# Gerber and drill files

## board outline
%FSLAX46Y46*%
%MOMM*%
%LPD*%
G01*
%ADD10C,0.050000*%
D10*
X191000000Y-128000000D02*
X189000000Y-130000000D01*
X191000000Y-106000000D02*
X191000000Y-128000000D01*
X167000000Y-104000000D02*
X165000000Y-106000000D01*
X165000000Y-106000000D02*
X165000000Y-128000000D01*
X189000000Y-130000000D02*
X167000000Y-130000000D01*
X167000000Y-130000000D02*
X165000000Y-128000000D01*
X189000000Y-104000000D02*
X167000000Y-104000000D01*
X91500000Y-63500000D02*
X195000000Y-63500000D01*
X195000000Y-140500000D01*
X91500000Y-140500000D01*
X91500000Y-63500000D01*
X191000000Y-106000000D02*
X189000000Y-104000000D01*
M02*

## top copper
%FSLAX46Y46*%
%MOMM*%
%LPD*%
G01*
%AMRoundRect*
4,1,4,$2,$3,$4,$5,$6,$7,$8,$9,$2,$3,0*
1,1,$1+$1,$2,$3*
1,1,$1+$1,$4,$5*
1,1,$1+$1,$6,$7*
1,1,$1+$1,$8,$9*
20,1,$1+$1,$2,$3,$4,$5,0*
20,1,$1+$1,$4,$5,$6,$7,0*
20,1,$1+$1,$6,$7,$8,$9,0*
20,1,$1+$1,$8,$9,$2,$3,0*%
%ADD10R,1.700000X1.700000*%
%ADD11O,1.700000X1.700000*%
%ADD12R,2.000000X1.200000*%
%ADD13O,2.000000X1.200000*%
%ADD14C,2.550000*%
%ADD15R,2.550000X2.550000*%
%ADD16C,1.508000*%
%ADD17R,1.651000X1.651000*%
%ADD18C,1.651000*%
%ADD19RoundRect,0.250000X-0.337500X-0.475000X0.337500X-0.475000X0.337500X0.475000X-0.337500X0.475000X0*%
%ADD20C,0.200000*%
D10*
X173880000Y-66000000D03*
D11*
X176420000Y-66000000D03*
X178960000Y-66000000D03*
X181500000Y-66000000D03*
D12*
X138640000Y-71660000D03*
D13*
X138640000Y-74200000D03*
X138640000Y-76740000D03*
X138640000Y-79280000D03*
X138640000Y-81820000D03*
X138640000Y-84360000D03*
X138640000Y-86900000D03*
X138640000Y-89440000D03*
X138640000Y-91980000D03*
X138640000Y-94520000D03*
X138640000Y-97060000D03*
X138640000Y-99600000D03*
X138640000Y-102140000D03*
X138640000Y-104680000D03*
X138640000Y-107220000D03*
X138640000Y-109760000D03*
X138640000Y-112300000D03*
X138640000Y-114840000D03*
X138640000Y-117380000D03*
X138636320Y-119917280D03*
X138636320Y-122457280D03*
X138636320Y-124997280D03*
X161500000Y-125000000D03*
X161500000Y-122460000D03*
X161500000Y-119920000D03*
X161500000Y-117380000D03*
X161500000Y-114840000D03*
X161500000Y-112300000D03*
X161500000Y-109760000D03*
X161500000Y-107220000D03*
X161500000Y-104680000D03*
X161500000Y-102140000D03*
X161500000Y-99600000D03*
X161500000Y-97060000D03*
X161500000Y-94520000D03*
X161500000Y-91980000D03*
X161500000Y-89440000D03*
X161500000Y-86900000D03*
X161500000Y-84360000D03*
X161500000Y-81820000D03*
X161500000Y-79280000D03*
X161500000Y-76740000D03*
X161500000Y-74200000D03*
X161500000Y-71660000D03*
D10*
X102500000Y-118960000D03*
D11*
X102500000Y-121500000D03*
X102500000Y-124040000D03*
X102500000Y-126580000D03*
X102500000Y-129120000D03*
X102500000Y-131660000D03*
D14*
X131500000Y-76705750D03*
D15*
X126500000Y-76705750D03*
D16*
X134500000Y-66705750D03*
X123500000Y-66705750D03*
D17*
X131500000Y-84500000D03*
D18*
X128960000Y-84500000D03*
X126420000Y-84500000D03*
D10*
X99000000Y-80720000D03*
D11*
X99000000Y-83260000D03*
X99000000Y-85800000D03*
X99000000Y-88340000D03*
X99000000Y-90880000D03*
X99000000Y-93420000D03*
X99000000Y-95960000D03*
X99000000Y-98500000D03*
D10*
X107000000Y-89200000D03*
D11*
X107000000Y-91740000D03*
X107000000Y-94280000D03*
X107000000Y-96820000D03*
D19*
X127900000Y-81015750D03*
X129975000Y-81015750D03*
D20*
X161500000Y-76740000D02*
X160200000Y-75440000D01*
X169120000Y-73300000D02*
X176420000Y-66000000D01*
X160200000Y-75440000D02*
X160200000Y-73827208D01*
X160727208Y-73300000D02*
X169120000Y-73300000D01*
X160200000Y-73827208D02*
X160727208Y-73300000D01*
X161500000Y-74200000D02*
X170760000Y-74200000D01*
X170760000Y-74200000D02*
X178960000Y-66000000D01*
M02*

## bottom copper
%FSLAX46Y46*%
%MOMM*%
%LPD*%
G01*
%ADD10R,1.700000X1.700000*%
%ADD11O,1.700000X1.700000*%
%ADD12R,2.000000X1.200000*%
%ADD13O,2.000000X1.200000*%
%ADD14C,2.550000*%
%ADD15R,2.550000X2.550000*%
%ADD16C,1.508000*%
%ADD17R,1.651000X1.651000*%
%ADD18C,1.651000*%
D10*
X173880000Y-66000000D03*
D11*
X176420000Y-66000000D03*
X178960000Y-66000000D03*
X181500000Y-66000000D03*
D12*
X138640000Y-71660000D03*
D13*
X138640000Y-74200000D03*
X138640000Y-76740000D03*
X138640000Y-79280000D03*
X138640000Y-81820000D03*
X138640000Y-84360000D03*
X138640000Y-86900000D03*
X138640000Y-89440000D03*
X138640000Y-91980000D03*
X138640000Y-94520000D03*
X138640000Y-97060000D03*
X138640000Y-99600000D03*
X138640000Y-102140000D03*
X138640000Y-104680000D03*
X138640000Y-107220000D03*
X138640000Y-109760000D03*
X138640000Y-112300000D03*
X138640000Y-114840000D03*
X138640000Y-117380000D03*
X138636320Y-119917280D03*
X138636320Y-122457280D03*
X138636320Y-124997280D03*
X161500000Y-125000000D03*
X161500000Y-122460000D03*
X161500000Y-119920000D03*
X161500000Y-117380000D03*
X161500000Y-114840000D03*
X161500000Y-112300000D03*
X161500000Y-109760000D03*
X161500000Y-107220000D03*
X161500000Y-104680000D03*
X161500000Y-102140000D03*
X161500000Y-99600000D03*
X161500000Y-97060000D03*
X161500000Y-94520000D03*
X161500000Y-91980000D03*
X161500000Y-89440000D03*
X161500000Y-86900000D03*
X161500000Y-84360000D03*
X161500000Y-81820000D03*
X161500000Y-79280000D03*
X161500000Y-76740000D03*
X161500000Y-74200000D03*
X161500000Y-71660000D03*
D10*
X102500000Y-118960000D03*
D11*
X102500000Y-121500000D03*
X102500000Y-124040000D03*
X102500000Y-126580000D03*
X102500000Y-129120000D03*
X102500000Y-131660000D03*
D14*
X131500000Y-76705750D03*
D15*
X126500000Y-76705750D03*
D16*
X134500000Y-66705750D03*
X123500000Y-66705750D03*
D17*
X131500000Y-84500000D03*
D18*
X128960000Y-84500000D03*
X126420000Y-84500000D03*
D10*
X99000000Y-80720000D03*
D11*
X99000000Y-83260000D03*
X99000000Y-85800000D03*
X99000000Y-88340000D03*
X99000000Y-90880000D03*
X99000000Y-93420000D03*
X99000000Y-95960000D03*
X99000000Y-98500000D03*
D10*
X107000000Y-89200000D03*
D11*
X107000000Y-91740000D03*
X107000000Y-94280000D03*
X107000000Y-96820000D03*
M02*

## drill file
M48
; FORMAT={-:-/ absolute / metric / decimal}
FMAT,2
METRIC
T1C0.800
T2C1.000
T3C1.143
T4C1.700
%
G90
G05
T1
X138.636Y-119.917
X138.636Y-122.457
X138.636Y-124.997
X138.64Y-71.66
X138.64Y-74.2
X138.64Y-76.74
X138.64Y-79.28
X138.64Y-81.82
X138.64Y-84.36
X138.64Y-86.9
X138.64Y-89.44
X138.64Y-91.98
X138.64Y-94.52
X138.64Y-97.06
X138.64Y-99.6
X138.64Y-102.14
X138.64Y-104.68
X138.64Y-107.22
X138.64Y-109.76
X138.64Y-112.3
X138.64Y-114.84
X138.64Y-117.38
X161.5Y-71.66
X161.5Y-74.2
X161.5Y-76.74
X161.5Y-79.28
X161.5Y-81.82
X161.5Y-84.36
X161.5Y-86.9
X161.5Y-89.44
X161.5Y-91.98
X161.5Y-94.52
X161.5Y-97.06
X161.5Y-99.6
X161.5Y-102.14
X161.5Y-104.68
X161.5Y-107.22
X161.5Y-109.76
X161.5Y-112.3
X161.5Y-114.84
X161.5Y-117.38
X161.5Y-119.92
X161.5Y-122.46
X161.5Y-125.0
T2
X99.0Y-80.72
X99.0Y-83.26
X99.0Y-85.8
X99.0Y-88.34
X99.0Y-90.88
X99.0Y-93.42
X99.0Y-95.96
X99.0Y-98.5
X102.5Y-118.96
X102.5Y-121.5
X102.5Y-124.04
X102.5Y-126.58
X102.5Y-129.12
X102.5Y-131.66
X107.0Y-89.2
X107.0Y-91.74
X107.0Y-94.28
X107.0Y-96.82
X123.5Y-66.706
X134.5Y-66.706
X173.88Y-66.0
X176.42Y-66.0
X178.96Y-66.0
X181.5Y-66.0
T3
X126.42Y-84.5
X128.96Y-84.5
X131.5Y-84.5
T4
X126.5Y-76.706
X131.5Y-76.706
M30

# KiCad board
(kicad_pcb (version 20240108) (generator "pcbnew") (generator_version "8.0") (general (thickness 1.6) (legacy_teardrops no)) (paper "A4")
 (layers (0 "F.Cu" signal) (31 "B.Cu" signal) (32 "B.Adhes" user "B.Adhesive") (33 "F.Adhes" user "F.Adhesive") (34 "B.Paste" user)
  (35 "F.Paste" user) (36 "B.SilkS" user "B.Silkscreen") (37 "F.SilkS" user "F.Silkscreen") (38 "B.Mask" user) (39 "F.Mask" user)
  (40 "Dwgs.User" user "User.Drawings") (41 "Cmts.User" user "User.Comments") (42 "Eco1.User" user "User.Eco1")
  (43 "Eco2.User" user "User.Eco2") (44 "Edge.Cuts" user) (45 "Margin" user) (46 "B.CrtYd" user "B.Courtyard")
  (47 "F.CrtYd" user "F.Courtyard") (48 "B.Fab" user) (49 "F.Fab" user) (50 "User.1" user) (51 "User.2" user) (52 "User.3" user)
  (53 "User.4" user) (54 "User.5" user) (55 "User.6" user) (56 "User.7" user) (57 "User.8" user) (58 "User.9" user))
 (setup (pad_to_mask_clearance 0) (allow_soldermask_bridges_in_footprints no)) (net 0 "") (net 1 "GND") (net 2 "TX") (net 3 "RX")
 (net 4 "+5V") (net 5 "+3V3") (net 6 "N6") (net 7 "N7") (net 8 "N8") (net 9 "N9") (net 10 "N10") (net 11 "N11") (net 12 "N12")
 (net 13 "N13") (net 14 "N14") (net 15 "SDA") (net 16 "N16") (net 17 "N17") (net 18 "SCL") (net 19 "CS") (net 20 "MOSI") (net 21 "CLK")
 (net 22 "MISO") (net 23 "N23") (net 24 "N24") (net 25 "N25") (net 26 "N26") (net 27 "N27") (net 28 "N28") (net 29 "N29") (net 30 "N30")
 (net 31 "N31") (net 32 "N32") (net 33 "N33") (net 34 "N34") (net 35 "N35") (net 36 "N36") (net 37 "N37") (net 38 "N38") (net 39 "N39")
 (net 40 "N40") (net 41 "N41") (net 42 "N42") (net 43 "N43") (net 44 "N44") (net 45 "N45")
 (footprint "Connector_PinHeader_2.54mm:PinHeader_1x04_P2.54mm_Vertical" (layer "F.Cu") (at 173.88 66 90)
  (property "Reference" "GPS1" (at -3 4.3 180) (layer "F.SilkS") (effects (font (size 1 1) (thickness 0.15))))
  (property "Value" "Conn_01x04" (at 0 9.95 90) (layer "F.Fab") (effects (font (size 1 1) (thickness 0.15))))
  (pad "1" thru_hole rect (at 0 0 90) (size 1.7 1.7) (drill 1) (layers "*.Cu" "*.Mask") (remove_unused_layers no) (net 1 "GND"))
  (pad "2" thru_hole oval (at 0 2.54 90) (size 1.7 1.7) (drill 1) (layers "*.Cu" "*.Mask") (remove_unused_layers no) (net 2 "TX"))
  (pad "3" thru_hole oval (at 0 5.08 90) (size 1.7 1.7) (drill 1) (layers "*.Cu" "*.Mask") (remove_unused_layers no) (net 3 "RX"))
  (pad "4" thru_hole oval (at 0 7.62 90) (size 1.7 1.7) (drill 1) (layers "*.Cu" "*.Mask") (remove_unused_layers no) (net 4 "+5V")))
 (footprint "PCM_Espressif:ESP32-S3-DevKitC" (layer "F.Cu") (at 138.64 71.66)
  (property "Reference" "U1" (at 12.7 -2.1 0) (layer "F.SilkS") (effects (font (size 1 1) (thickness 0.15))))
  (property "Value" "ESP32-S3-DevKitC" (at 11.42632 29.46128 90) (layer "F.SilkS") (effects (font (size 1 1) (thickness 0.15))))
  (pad "1" thru_hole rect (at 0 0 270) (size 1.2 2) (drill 0.8) (layers "*.Cu" "*.Mask") (remove_unused_layers no) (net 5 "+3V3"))
  (pad "2" thru_hole oval (at 0 2.54 270) (size 1.2 2) (drill 0.8) (layers "*.Cu" "*.Mask") (remove_unused_layers no) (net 5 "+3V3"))
  (pad "3" thru_hole oval (at 0 5.08 270) (size 1.2 2) (drill 0.8) (layers "*.Cu" "*.Mask") (remove_unused_layers no) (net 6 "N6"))
  (pad "4" thru_hole oval (at 0 7.62 270) (size 1.2 2) (drill 0.8) (layers "*.Cu" "*.Mask") (remove_unused_layers no) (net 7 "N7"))
  (pad "5" thru_hole oval (at 0 10.16 270) (size 1.2 2) (drill 0.8) (layers "*.Cu" "*.Mask") (remove_unused_layers no) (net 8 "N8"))
  (pad "6" thru_hole oval (at 0 12.7 270) (size 1.2 2) (drill 0.8) (layers "*.Cu" "*.Mask") (remove_unused_layers no) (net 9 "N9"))
  (pad "7" thru_hole oval (at 0 15.24 270) (size 1.2 2) (drill 0.8) (layers "*.Cu" "*.Mask") (remove_unused_layers no) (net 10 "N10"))
  (pad "8" thru_hole oval (at 0 17.78 270) (size 1.2 2) (drill 0.8) (layers "*.Cu" "*.Mask") (remove_unused_layers no) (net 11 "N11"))
  (pad "9" thru_hole oval (at 0 20.32 270) (size 1.2 2) (drill 0.8) (layers "*.Cu" "*.Mask") (remove_unused_layers no) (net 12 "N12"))
  (pad "10" thru_hole oval (at 0 22.86 270) (size 1.2 2) (drill 0.8) (layers "*.Cu" "*.Mask") (remove_unused_layers no) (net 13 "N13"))
  (pad "11" thru_hole oval (at 0 25.4 270) (size 1.2 2) (drill 0.8) (layers "*.Cu" "*.Mask") (remove_unused_layers no) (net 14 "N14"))
  (pad "12" thru_hole oval (at 0 27.94 270) (size 1.2 2) (drill 0.8) (layers "*.Cu" "*.Mask") (remove_unused_layers no) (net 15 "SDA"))
  (pad "13" thru_hole oval (at 0 30.48 270) (size 1.2 2) (drill 0.8) (layers "*.Cu" "*.Mask") (remove_unused_layers no) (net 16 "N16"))
  (pad "14" thru_hole oval (at 0 33.02 270) (size 1.2 2) (drill 0.8) (layers "*.Cu" "*.Mask") (remove_unused_layers no) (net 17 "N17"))
  (pad "15" thru_hole oval (at 0 35.56 270) (size 1.2 2) (drill 0.8) (layers "*.Cu" "*.Mask") (remove_unused_layers no) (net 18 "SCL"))
  (pad "16" thru_hole oval (at 0 38.1 270) (size 1.2 2) (drill 0.8) (layers "*.Cu" "*.Mask") (remove_unused_layers no) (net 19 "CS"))
  (pad "17" thru_hole oval (at 0 40.64 270) (size 1.2 2) (drill 0.8) (layers "*.Cu" "*.Mask") (remove_unused_layers no) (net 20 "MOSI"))
  (pad "18" thru_hole oval (at 0 43.18 270) (size 1.2 2) (drill 0.8) (layers "*.Cu" "*.Mask") (remove_unused_layers no) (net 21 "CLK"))
  (pad "19" thru_hole oval (at 0 45.72 270) (size 1.2 2) (drill 0.8) (layers "*.Cu" "*.Mask") (remove_unused_layers no) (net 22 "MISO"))
  (pad "20" thru_hole oval (at -0.00368 48.25728 270) (size 1.2 2) (drill 0.8) (layers "*.Cu" "*.Mask") (remove_unused_layers no)
   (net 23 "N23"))
  (pad "21" thru_hole oval (at -0.00368 50.79728 270) (size 1.2 2) (drill 0.8) (layers "*.Cu" "*.Mask") (remove_unused_layers no)
   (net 4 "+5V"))
  (pad "22" thru_hole oval (at -0.00368 53.33728 270) (size 1.2 2) (drill 0.8) (layers "*.Cu" "*.Mask") (remove_unused_layers no)
   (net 1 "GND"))
  (pad "23" thru_hole oval (at 22.86 53.34 270) (size 1.2 2) (drill 0.8) (layers "*.Cu" "*.Mask") (remove_unused_layers no) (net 1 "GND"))
  (pad "24" thru_hole oval (at 22.86 50.8 270) (size 1.2 2) (drill 0.8) (layers "*.Cu" "*.Mask") (remove_unused_layers no) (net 1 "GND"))
  (pad "25" thru_hole oval (at 22.86 48.26 270) (size 1.2 2) (drill 0.8) (layers "*.Cu" "*.Mask") (remove_unused_layers no) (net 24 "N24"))
  (pad "26" thru_hole oval (at 22.86 45.72 270) (size 1.2 2) (drill 0.8) (layers "*.Cu" "*.Mask") (remove_unused_layers no) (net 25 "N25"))
  (pad "27" thru_hole oval (at 22.86 43.18 270) (size 1.2 2) (drill 0.8) (layers "*.Cu" "*.Mask") (remove_unused_layers no) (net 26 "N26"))
  (pad "28" thru_hole oval (at 22.86 40.64 270) (size 1.2 2) (drill 0.8) (layers "*.Cu" "*.Mask") (remove_unused_layers no) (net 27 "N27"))
  (pad "29" thru_hole oval (at 22.86 38.1 270) (size 1.2 2) (drill 0.8) (layers "*.Cu" "*.Mask") (remove_unused_layers no) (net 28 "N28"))
  (pad "30" thru_hole oval (at 22.86 35.56 270) (size 1.2 2) (drill 0.8) (layers "*.Cu" "*.Mask") (remove_unused_layers no) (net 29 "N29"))
  (pad "31" thru_hole oval (at 22.86 33.02 270) (size 1.2 2) (drill 0.8) (layers "*.Cu" "*.Mask") (remove_unused_layers no) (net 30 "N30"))
  (pad "32" thru_hole oval (at 22.86 30.48 270) (size 1.2 2) (drill 0.8) (layers "*.Cu" "*.Mask") (remove_unused_layers no) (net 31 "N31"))
  (pad "33" thru_hole oval (at 22.86 27.94 270) (size 1.2 2) (drill 0.8) (layers "*.Cu" "*.Mask") (remove_unused_layers no) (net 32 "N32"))
  (pad "34" thru_hole oval (at 22.86 25.4 270) (size 1.2 2) (drill 0.8) (layers "*.Cu" "*.Mask") (remove_unused_layers no) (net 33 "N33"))
  (pad "35" thru_hole oval (at 22.86 22.86 270) (size 1.2 2) (drill 0.8) (layers "*.Cu" "*.Mask") (remove_unused_layers no) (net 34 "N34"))
  (pad "36" thru_hole oval (at 22.86 20.32 270) (size 1.2 2) (drill 0.8) (layers "*.Cu" "*.Mask") (remove_unused_layers no) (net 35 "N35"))
  (pad "37" thru_hole oval (at 22.86 17.78 270) (size 1.2 2) (drill 0.8) (layers "*.Cu" "*.Mask") (remove_unused_layers no) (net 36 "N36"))
  (pad "38" thru_hole oval (at 22.86 15.24 270) (size 1.2 2) (drill 0.8) (layers "*.Cu" "*.Mask") (remove_unused_layers no) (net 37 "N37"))
  (pad "39" thru_hole oval (at 22.86 12.7 270) (size 1.2 2) (drill 0.8) (layers "*.Cu" "*.Mask") (remove_unused_layers no) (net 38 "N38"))
  (pad "40" thru_hole oval (at 22.86 10.16 270) (size 1.2 2) (drill 0.8) (layers "*.Cu" "*.Mask") (remove_unused_layers no) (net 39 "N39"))
  (pad "41" thru_hole oval (at 22.86 7.62 270) (size 1.2 2) (drill 0.8) (layers "*.Cu" "*.Mask") (remove_unused_layers no) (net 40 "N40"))
  (pad "42" thru_hole oval (at 22.86 5.08 270) (size 1.2 2) (drill 0.8) (layers "*.Cu" "*.Mask") (remove_unused_layers no) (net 2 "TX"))
  (pad "43" thru_hole oval (at 22.86 2.54 270) (size 1.2 2) (drill 0.8) (layers "*.Cu" "*.Mask") (remove_unused_layers no) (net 3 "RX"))
  (pad "44" thru_hole oval (at 22.86 0 270) (size 1.2 2) (drill 0.8) (layers "*.Cu" "*.Mask") (remove_unused_layers no) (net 1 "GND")))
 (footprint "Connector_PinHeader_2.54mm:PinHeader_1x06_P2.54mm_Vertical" (layer "F.Cu") (at 102.5 118.96)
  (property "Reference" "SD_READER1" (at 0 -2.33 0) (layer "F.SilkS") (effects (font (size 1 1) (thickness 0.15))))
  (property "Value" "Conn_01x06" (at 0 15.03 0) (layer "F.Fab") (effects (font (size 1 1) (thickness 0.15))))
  (pad "1" thru_hole rect (at 0 0) (size 1.7 1.7) (drill 1) (layers "*.Cu" "*.Mask") (remove_unused_layers no) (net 1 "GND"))
  (pad "2" thru_hole oval (at 0 2.54) (size 1.7 1.7) (drill 1) (layers "*.Cu" "*.Mask") (remove_unused_layers no) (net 19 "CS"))
  (pad "3" thru_hole oval (at 0 5.08) (size 1.7 1.7) (drill 1) (layers "*.Cu" "*.Mask") (remove_unused_layers no) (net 20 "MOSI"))
  (pad "4" thru_hole oval (at 0 7.62) (size 1.7 1.7) (drill 1) (layers "*.Cu" "*.Mask") (remove_unused_layers no) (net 21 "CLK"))
  (pad "5" thru_hole oval (at 0 10.16) (size 1.7 1.7) (drill 1) (layers "*.Cu" "*.Mask") (remove_unused_layers no) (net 22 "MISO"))
  (pad "6" thru_hole oval (at 0 12.7) (size 1.7 1.7) (drill 1) (layers "*.Cu" "*.Mask") (remove_unused_layers no) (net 5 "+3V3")))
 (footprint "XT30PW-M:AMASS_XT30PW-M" (layer "F.Cu") (at 129 66.70575)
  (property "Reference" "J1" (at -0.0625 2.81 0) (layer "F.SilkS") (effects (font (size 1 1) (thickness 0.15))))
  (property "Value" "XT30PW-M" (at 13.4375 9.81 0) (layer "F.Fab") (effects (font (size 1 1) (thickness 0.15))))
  (pad "N" thru_hole circle (at 2.5 10) (size 2.55 2.55) (drill 1.7) (layers "*.Cu" "*.Mask") (remove_unused_layers no) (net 1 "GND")
   (solder_mask_margin 0.102))
  (pad "P" thru_hole rect (at -2.5 10) (size 2.55 2.55) (drill 1.7) (layers "*.Cu" "*.Mask") (remove_unused_layers no) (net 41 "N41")
   (solder_mask_margin 0.102))
  (pad "S1" thru_hole circle (at 5.5 0) (size 1.508 1.508) (drill 1) (layers "*.Cu" "*.Mask") (remove_unused_layers no)
   (solder_mask_margin 0.102))
  (pad "S2" thru_hole circle (at -5.5 0) (size 1.508 1.508) (drill 1) (layers "*.Cu" "*.Mask") (remove_unused_layers no)
   (solder_mask_margin 0.102)))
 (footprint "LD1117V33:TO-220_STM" (layer "F.Cu") (at 131.5 84.5 180)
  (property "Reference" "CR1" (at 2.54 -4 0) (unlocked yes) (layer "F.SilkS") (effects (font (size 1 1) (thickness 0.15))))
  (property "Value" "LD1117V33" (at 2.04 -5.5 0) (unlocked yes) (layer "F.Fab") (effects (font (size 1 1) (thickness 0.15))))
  (pad "1" thru_hole rect (at 0 0 180) (size 1.651 1.651) (drill 1.143) (layers "*.Cu" "*.Mask") (remove_unused_layers no) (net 1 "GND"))
  (pad "2" thru_hole circle (at 2.54 0 180) (size 1.651 1.651) (drill 1.143) (layers "*.Cu" "*.Mask") (remove_unused_layers no)
   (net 5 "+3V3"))
  (pad "3" thru_hole circle (at 5.08 0 180) (size 1.651 1.651) (drill 1.143) (layers "*.Cu" "*.Mask") (remove_unused_layers no)
   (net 41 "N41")))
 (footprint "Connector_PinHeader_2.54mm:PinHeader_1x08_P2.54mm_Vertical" (layer "F.Cu") (at 99 80.72)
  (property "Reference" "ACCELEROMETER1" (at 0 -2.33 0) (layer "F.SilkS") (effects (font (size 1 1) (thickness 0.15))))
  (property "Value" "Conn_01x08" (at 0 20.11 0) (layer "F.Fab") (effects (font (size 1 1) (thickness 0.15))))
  (pad "1" thru_hole rect (at 0 0) (size 1.7 1.7) (drill 1) (layers "*.Cu" "*.Mask") (remove_unused_layers no) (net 4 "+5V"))
  (pad "2" thru_hole oval (at 0 2.54) (size 1.7 1.7) (drill 1) (layers "*.Cu" "*.Mask") (remove_unused_layers no) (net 1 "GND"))
  (pad "3" thru_hole oval (at 0 5.08) (size 1.7 1.7) (drill 1) (layers "*.Cu" "*.Mask") (remove_unused_layers no) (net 18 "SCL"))
  (pad "4" thru_hole oval (at 0 7.62) (size 1.7 1.7) (drill 1) (layers "*.Cu" "*.Mask") (remove_unused_layers no) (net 15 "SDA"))
  (pad "5" thru_hole oval (at 0 10.16) (size 1.7 1.7) (drill 1) (layers "*.Cu" "*.Mask") (remove_unused_layers no) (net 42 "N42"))
  (pad "6" thru_hole oval (at 0 12.7) (size 1.7 1.7) (drill 1) (layers "*.Cu" "*.Mask") (remove_unused_layers no) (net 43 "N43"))
  (pad "7" thru_hole oval (at 0 15.24) (size 1.7 1.7) (drill 1) (layers "*.Cu" "*.Mask") (remove_unused_layers no) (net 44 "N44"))
  (pad "8" thru_hole oval (at 0 17.78) (size 1.7 1.7) (drill 1) (layers "*.Cu" "*.Mask") (remove_unused_layers no) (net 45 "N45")))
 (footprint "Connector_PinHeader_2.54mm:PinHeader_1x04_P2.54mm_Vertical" (layer "F.Cu") (at 107 89.2)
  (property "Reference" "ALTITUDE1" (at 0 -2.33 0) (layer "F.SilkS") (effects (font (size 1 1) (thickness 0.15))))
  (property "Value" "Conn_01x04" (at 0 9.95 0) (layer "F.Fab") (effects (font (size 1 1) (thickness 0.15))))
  (pad "1" thru_hole rect (at 0 0) (size 1.7 1.7) (drill 1) (layers "*.Cu" "*.Mask") (remove_unused_layers no) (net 5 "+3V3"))
  (pad "2" thru_hole oval (at 0 2.54) (size 1.7 1.7) (drill 1) (layers "*.Cu" "*.Mask") (remove_unused_layers no) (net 1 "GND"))
  (pad "3" thru_hole oval (at 0 5.08) (size 1.7 1.7) (drill 1) (layers "*.Cu" "*.Mask") (remove_unused_layers no) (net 18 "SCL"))
  (pad "4" thru_hole oval (at 0 7.62) (size 1.7 1.7) (drill 1) (layers "*.Cu" "*.Mask") (remove_unused_layers no) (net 15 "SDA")))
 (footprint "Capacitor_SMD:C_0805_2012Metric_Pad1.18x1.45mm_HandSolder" (layer "F.Cu") (at 128.9375 81.01575)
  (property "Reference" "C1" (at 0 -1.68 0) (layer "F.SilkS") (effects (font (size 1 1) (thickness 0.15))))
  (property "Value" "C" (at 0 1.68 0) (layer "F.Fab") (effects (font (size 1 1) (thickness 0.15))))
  (pad "1" smd roundrect (at -1.0375 0) (size 1.175 1.45) (layers "F.Cu" "F.Paste" "F.Mask") (roundrect_rratio 0.212766) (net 41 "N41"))
  (pad "2" smd roundrect (at 1.0375 0) (size 1.175 1.45) (layers "F.Cu" "F.Paste" "F.Mask") (roundrect_rratio 0.212766) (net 1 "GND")))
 (gr_line (start 191 128) (end 189 130) (stroke (width 0.05) (type default)) (layer "Edge.Cuts"))
 (gr_line (start 191 106) (end 191 128) (stroke (width 0.05) (type default)) (layer "Edge.Cuts"))
 (gr_line (start 167 104) (end 165 106) (stroke (width 0.05) (type default)) (layer "Edge.Cuts"))
 (gr_line (start 165 106) (end 165 128) (stroke (width 0.05) (type default)) (layer "Edge.Cuts"))
 (gr_line (start 189 130) (end 167 130) (stroke (width 0.05) (type default)) (layer "Edge.Cuts"))
 (gr_line (start 167 130) (end 165 128) (stroke (width 0.05) (type default)) (layer "Edge.Cuts"))
 (gr_line (start 189 104) (end 167 104) (stroke (width 0.05) (type default)) (layer "Edge.Cuts"))
 (gr_rect (start 91.5 63.5) (end 195 140.5) (stroke (width 0.05) (type default)) (fill none) (layer "Edge.Cuts"))
 (gr_line (start 191 106) (end 189 104) (stroke (width 0.05) (type default)) (layer "Edge.Cuts"))
 (segment (start 161.5 76.74) (end 160.2 75.44) (width 0.2) (layer "F.Cu") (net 2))
 (segment (start 169.12 73.3) (end 176.42 66) (width 0.2) (layer "F.Cu") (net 2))
 (segment (start 160.2 75.44) (end 160.2 73.827208) (width 0.2) (layer "F.Cu") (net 2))
 (segment (start 160.727208 73.3) (end 169.12 73.3) (width 0.2) (layer "F.Cu") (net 2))
 (segment (start 160.2 73.827208) (end 160.727208 73.3) (width 0.2) (layer "F.Cu") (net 2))
 (segment (start 161.5 74.2) (end 170.76 74.2) (width 0.2) (layer "F.Cu") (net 3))
 (segment (start 170.76 74.2) (end 178.96 66) (width 0.2) (layer "F.Cu") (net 3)))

